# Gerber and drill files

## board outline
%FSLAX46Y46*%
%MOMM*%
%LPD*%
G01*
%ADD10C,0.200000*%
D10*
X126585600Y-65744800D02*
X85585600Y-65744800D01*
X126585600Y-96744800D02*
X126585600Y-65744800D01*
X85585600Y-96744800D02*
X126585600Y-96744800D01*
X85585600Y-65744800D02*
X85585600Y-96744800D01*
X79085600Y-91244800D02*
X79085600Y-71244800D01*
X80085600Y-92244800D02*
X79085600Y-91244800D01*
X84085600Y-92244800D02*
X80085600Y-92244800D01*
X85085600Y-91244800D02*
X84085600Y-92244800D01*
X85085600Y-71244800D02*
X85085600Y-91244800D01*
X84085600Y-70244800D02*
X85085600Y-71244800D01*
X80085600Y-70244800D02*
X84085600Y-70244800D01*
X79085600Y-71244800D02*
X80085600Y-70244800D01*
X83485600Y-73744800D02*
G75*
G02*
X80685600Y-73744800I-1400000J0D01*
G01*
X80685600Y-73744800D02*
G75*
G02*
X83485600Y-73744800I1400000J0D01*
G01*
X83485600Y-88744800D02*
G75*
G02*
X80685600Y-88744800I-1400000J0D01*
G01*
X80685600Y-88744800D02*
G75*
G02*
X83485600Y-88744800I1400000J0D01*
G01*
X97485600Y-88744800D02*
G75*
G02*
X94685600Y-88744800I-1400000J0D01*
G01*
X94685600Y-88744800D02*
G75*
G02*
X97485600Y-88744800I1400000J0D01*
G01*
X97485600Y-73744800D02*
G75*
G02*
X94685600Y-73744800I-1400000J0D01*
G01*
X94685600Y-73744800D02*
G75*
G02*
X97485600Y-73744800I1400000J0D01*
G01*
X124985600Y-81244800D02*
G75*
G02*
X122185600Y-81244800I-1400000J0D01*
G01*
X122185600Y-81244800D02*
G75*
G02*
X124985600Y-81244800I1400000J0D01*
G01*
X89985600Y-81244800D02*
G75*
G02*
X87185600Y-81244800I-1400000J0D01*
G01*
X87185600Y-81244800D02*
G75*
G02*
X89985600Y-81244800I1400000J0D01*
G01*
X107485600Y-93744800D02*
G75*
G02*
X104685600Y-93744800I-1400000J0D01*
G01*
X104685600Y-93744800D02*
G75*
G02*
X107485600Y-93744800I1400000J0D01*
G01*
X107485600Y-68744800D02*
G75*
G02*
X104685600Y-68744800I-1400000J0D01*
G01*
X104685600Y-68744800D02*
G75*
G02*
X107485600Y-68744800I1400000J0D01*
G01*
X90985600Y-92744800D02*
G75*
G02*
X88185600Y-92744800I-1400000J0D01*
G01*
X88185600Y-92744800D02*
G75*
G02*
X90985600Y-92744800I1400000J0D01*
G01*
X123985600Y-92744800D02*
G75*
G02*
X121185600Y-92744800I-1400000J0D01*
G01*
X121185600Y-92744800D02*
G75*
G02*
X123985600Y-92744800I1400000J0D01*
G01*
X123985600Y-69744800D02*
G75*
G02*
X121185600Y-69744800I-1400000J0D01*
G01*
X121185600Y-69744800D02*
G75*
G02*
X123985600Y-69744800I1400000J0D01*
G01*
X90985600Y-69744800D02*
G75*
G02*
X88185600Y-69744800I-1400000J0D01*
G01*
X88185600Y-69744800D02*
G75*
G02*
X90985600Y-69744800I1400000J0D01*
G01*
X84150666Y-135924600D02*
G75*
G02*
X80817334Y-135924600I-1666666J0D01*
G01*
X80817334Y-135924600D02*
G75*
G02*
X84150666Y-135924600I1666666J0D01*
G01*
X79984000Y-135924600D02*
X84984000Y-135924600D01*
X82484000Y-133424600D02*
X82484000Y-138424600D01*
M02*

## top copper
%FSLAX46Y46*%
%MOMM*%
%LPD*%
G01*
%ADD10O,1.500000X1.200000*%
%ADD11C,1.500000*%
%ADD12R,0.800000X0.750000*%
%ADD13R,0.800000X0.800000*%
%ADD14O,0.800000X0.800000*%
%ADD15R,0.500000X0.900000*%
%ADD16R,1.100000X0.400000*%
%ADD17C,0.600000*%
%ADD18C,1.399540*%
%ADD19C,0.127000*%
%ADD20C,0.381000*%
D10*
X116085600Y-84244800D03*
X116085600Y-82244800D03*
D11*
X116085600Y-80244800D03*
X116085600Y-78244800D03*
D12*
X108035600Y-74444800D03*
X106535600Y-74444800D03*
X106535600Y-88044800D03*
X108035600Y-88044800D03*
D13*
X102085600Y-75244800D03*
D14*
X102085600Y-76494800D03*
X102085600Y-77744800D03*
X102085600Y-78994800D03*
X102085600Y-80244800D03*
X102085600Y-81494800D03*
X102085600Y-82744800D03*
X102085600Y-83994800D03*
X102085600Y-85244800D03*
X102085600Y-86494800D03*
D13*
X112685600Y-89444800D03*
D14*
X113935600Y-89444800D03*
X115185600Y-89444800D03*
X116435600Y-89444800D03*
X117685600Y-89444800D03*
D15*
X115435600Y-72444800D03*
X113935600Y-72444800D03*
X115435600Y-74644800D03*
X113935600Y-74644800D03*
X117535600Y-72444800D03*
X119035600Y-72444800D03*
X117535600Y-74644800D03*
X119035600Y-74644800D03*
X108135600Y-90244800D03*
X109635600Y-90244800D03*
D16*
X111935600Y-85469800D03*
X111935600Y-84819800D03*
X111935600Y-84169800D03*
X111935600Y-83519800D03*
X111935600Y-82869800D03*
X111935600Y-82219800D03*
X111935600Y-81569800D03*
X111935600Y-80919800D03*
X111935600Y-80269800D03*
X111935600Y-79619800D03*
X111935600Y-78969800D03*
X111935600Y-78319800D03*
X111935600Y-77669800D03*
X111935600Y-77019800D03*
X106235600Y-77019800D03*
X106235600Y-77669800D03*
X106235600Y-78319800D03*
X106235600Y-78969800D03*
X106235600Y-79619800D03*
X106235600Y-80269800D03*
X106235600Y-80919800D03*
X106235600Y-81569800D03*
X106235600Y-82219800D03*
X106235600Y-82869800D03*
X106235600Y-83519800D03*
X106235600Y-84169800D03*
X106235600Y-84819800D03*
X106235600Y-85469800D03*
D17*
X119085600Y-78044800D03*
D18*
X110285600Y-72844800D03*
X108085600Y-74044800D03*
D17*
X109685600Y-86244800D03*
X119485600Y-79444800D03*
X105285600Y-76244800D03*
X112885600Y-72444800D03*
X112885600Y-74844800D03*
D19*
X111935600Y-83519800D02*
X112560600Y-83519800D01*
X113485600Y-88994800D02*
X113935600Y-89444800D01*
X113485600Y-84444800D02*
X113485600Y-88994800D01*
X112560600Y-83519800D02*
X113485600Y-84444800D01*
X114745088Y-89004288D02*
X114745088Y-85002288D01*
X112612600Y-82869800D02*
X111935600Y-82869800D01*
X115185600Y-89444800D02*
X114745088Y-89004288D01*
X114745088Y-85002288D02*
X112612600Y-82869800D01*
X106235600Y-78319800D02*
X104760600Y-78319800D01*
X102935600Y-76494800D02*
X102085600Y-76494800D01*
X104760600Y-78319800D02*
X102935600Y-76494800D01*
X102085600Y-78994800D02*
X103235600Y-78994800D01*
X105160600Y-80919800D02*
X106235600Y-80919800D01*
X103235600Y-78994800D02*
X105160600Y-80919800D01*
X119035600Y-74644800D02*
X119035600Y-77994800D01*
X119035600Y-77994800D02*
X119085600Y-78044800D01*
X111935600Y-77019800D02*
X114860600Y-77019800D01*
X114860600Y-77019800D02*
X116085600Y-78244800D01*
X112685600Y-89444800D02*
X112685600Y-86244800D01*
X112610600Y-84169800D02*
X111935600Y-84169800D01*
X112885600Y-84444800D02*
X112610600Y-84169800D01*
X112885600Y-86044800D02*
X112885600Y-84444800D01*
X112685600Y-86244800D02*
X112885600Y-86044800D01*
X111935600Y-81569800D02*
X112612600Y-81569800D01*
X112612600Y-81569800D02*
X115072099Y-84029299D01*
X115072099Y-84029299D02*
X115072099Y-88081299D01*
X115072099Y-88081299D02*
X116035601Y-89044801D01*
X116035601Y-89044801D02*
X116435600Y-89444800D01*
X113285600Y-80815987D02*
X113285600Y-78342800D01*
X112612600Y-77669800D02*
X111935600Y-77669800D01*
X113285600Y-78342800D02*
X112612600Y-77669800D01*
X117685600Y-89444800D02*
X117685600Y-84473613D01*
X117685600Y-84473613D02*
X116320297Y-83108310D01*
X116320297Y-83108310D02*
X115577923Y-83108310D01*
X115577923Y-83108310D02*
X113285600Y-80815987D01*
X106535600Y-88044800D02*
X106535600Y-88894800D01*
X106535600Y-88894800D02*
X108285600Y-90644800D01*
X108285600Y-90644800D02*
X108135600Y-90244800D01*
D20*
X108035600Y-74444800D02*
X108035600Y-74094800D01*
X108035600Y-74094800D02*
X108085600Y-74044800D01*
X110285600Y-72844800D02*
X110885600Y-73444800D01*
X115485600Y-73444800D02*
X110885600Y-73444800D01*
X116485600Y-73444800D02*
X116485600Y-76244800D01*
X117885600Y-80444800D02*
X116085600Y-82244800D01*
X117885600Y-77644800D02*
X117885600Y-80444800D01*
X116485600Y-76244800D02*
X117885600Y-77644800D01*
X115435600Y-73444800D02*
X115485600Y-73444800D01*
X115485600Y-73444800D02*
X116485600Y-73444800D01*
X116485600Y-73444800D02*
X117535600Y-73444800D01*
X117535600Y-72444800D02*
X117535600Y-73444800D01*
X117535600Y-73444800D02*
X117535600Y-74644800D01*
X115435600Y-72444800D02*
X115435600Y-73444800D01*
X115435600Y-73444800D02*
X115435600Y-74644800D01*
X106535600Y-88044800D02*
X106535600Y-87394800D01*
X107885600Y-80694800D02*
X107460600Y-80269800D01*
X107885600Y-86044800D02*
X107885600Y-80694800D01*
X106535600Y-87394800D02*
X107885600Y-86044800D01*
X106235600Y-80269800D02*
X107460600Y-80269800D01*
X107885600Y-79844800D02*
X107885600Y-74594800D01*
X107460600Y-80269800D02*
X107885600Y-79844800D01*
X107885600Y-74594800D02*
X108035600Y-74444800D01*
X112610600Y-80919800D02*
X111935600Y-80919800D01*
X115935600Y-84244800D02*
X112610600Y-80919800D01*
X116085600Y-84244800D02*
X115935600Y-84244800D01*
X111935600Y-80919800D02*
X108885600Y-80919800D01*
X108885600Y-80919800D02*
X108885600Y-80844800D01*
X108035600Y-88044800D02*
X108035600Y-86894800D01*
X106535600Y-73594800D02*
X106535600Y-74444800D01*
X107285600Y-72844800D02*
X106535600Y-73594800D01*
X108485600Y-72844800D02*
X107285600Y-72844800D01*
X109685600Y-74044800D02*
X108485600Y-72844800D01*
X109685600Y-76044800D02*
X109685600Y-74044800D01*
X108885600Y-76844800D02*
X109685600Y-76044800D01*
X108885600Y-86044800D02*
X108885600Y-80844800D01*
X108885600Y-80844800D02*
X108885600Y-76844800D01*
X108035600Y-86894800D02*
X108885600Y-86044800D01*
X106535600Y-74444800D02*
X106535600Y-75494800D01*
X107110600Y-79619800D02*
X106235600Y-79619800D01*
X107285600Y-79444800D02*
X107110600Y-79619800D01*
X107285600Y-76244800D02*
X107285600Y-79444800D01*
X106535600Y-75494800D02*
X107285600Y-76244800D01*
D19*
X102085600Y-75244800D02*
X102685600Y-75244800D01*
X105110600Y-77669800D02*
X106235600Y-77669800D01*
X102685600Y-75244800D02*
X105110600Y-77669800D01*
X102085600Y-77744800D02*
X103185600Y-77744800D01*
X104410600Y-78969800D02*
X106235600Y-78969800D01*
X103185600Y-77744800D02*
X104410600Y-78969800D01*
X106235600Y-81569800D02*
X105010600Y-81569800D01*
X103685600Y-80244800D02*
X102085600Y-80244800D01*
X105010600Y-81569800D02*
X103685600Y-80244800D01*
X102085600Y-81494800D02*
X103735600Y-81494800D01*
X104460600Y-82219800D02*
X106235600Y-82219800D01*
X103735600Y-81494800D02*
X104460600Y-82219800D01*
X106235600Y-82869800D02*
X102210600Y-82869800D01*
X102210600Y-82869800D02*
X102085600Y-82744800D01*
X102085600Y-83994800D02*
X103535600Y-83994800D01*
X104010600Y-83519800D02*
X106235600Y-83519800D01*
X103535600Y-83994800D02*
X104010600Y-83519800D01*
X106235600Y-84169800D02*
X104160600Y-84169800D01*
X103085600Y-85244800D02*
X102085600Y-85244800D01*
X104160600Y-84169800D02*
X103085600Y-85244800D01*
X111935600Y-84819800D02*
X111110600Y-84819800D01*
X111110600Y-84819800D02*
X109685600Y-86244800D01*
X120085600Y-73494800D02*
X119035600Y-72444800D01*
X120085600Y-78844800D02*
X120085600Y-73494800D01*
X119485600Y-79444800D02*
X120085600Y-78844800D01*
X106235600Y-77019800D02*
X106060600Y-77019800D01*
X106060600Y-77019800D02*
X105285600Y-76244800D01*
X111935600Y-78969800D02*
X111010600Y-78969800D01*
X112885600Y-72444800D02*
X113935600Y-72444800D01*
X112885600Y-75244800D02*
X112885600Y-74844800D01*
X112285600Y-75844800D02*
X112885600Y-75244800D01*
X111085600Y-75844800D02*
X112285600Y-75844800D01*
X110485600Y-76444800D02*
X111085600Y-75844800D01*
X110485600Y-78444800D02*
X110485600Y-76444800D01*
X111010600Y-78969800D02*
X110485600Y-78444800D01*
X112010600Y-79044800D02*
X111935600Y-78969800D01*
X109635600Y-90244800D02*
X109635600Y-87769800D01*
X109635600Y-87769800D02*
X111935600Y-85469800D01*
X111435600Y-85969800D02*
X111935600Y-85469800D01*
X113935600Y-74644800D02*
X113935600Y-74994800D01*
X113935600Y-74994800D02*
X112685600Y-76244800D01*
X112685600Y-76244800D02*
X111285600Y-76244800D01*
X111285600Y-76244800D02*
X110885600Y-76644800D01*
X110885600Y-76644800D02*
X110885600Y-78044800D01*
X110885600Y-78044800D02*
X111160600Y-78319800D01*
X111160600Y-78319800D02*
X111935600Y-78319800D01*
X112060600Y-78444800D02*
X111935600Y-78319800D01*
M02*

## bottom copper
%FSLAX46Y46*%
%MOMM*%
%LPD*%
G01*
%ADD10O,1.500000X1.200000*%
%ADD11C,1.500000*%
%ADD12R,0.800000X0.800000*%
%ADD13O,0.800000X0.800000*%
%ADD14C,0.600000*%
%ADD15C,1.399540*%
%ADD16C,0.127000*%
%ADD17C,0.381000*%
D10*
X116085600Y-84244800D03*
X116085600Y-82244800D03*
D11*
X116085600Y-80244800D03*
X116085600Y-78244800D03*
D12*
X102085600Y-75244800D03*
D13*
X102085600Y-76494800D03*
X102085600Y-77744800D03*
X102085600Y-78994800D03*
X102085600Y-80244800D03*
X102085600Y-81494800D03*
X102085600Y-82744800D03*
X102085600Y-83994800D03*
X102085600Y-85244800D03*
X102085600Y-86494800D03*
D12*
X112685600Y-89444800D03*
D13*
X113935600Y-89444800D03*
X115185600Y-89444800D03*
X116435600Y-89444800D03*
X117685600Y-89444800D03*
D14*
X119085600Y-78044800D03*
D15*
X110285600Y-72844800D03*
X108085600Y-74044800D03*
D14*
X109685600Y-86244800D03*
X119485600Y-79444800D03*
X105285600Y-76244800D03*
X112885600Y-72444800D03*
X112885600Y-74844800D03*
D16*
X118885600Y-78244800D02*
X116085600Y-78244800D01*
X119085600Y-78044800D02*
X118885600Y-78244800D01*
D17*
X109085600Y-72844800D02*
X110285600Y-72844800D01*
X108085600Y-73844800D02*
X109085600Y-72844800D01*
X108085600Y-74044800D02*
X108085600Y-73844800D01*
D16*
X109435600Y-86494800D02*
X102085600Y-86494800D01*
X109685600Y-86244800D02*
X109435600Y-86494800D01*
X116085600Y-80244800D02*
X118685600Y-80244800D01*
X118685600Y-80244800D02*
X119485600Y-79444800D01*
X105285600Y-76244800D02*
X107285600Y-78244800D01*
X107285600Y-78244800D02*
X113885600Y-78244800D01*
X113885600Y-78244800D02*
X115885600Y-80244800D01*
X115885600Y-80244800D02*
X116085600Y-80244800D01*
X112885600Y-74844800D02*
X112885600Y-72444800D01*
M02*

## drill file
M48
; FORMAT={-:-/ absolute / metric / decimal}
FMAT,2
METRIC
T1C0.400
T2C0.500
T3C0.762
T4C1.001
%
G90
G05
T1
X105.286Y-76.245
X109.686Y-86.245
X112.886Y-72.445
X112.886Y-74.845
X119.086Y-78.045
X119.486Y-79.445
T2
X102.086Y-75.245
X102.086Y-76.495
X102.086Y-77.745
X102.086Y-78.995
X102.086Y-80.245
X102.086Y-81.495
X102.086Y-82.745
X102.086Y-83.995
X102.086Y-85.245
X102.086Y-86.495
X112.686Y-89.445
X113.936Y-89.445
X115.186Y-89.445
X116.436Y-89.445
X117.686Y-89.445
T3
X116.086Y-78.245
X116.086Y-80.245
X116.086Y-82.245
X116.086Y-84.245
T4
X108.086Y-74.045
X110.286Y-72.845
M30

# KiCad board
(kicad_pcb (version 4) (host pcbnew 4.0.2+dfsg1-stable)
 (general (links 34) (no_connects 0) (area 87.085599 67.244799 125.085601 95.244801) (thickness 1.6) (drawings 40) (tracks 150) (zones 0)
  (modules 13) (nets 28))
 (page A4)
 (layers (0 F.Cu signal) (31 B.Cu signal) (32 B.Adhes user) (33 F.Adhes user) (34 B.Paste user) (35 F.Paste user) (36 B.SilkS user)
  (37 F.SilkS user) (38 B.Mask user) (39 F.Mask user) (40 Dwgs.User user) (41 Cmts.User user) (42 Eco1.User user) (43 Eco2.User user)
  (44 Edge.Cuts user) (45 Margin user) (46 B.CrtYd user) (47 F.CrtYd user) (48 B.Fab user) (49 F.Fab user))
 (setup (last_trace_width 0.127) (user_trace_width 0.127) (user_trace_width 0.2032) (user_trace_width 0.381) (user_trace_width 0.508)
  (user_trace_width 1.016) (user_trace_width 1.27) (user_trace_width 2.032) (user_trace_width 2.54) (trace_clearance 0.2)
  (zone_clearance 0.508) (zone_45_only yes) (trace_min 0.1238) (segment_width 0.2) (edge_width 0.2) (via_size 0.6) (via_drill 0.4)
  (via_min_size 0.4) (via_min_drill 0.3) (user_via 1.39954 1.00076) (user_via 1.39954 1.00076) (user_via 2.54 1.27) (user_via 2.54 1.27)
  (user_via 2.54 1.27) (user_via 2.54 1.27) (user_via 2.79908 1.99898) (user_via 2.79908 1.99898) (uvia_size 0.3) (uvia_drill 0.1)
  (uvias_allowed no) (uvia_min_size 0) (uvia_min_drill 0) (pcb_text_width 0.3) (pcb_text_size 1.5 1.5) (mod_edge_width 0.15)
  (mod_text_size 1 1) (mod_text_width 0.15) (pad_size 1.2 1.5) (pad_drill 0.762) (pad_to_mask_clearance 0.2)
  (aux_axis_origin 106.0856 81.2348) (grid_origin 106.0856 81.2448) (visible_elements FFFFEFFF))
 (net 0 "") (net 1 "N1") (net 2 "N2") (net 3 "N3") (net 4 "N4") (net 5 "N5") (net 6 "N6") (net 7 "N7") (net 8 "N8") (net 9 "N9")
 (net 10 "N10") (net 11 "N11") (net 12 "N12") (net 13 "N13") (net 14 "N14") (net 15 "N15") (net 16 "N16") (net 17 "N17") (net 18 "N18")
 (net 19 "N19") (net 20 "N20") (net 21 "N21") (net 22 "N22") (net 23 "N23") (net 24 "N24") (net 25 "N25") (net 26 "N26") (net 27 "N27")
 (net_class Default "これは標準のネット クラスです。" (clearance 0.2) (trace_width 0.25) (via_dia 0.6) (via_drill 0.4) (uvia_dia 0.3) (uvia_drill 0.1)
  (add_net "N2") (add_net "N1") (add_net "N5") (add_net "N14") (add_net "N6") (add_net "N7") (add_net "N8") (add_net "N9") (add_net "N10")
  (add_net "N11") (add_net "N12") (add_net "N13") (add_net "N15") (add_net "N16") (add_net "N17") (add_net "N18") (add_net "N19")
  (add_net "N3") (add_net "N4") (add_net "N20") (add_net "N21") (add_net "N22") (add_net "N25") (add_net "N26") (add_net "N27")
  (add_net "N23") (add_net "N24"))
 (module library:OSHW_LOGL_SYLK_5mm (layer F.Cu) (at 82.0856 81.2448 270)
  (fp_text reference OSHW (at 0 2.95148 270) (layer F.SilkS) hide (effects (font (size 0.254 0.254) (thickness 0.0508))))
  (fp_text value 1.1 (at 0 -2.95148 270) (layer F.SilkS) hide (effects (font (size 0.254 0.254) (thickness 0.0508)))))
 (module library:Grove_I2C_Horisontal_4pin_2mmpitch (layer F.Cu) (at 116.0856 81.2448 90)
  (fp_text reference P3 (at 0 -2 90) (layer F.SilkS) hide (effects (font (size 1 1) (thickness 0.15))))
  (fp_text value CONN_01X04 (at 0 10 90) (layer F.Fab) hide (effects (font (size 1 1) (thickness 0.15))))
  (pad 1 thru_hole oval (at -3 0 90) (size 1.2 1.5) (drill 0.762) (layers *.Cu *.Mask F.SilkS) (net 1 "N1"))
  (pad 2 thru_hole oval (at -1 0 90) (size 1.2 1.5) (drill 0.762) (layers *.Cu *.Mask F.SilkS) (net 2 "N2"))
  (pad 3 thru_hole circle (at 1 0 90) (size 1.5 1.5) (drill 0.762) (layers *.Cu *.Mask F.SilkS) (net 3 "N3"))
  (pad 4 thru_hole circle (at 3 0 90) (size 1.5 1.5) (drill 0.762) (layers *.Cu *.Mask F.SilkS) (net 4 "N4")))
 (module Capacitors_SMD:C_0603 (layer F.Cu) (at 107.2856 74.4448 180)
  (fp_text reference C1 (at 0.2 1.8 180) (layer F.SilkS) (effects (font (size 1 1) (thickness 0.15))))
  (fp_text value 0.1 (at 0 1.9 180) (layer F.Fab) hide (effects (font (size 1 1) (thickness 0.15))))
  (pad 1 smd rect (at -0.75 0 180) (size 0.8 0.75) (layers F.Cu F.Paste F.Mask) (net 2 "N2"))
  (pad 2 smd rect (at 0.75 0 180) (size 0.8 0.75) (layers F.Cu F.Paste F.Mask) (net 1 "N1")))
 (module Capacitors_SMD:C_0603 (layer F.Cu) (at 107.2856 88.0448)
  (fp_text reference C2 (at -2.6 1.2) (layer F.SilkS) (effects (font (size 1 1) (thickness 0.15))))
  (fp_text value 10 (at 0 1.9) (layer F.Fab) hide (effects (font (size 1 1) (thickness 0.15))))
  (pad 1 smd rect (at -0.75 0) (size 0.8 0.75) (layers F.Cu F.Paste F.Mask) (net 2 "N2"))
  (pad 2 smd rect (at 0.75 0) (size 0.8 0.75) (layers F.Cu F.Paste F.Mask) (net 1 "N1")))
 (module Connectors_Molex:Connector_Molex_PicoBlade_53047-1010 (layer F.Cu) (at 102.0856 75.2448 270)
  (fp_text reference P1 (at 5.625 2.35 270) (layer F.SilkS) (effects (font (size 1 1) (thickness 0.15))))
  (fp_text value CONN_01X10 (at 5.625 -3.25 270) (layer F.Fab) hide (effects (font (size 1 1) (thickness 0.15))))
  (pad 1 thru_hole rect (at 0 0 270) (size 0.8 0.8) (drill 0.5) (layers *.Cu *.Mask F.SilkS) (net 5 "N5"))
  (pad 2 thru_hole oval (at 1.25 0 270) (size 0.8 0.8) (drill 0.5) (layers *.Cu *.Mask F.SilkS) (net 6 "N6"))
  (pad 3 thru_hole oval (at 2.5 0 270) (size 0.8 0.8) (drill 0.5) (layers *.Cu *.Mask F.SilkS) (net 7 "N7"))
  (pad 4 thru_hole oval (at 3.75 0 270) (size 0.8 0.8) (drill 0.5) (layers *.Cu *.Mask F.SilkS) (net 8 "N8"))
  (pad 5 thru_hole oval (at 5 0 270) (size 0.8 0.8) (drill 0.5) (layers *.Cu *.Mask F.SilkS) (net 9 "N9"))
  (pad 6 thru_hole oval (at 6.25 0 270) (size 0.8 0.8) (drill 0.5) (layers *.Cu *.Mask F.SilkS) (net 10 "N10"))
  (pad 7 thru_hole oval (at 7.5 0 270) (size 0.8 0.8) (drill 0.5) (layers *.Cu *.Mask F.SilkS) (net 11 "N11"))
  (pad 8 thru_hole oval (at 8.75 0 270) (size 0.8 0.8) (drill 0.5) (layers *.Cu *.Mask F.SilkS) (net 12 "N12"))
  (pad 9 thru_hole oval (at 10 0 270) (size 0.8 0.8) (drill 0.5) (layers *.Cu *.Mask F.SilkS) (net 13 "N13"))
  (pad 10 thru_hole oval (at 11.25 0 270) (size 0.8 0.8) (drill 0.5) (layers *.Cu *.Mask F.SilkS) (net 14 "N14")))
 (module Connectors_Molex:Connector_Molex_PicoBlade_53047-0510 (layer F.Cu) (at 112.6856 89.4448)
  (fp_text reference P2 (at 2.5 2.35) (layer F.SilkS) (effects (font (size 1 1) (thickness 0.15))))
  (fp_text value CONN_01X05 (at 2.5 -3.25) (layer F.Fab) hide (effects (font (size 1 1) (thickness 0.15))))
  (pad 1 thru_hole rect (at 0 0) (size 0.8 0.8) (drill 0.5) (layers *.Cu *.Mask F.SilkS) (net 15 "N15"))
  (pad 2 thru_hole oval (at 1.25 0) (size 0.8 0.8) (drill 0.5) (layers *.Cu *.Mask F.SilkS) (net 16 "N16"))
  (pad 3 thru_hole oval (at 2.5 0) (size 0.8 0.8) (drill 0.5) (layers *.Cu *.Mask F.SilkS) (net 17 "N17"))
  (pad 4 thru_hole oval (at 3.75 0) (size 0.8 0.8) (drill 0.5) (layers *.Cu *.Mask F.SilkS) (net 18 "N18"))
  (pad 5 thru_hole oval (at 5 0) (size 0.8 0.8) (drill 0.5) (layers *.Cu *.Mask F.SilkS) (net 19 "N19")))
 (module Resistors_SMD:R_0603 (layer F.Cu) (at 114.6856 72.4448 180)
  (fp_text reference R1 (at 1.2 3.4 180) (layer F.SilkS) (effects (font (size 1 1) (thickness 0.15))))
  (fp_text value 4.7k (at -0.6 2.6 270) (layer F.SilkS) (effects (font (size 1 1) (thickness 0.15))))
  (pad 1 smd rect (at -0.75 0 180) (size 0.5 0.9) (layers F.Cu F.Paste F.Mask) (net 2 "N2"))
  (pad 2 smd rect (at 0.75 0 180) (size 0.5 0.9) (layers F.Cu F.Paste F.Mask) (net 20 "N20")))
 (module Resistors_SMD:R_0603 (layer F.Cu) (at 114.6856 74.6448 180)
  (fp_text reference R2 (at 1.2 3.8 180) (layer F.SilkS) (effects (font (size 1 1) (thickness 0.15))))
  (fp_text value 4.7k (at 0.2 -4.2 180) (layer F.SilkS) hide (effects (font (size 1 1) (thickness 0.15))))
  (pad 1 smd rect (at -0.75 0 180) (size 0.5 0.9) (layers F.Cu F.Paste F.Mask) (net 2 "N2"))
  (pad 2 smd rect (at 0.75 0 180) (size 0.5 0.9) (layers F.Cu F.Paste F.Mask) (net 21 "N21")))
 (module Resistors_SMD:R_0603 (layer F.Cu) (at 118.2856 72.4448)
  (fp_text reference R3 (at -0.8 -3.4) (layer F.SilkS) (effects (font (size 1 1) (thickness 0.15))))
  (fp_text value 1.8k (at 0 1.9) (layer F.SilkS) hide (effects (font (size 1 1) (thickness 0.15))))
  (pad 1 smd rect (at -0.75 0) (size 0.5 0.9) (layers F.Cu F.Paste F.Mask) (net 2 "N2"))
  (pad 2 smd rect (at 0.75 0) (size 0.5 0.9) (layers F.Cu F.Paste F.Mask) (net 3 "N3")))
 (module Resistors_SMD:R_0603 (layer F.Cu) (at 118.2856 74.6448)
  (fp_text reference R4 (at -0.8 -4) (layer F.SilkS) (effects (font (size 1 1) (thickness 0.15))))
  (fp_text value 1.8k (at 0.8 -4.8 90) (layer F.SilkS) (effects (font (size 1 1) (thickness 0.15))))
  (pad 1 smd rect (at -0.75 0) (size 0.5 0.9) (layers F.Cu F.Paste F.Mask) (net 2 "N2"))
  (pad 2 smd rect (at 0.75 0) (size 0.5 0.9) (layers F.Cu F.Paste F.Mask) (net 4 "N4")))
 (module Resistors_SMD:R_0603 (layer F.Cu) (at 108.8856 90.2448)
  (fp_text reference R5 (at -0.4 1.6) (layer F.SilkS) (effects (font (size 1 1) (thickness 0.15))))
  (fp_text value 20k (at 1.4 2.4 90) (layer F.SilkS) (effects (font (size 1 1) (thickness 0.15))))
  (pad 1 smd rect (at -0.75 0) (size 0.5 0.9) (layers F.Cu F.Paste F.Mask) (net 2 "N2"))
  (pad 2 smd rect (at 0.75 0) (size 0.5 0.9) (layers F.Cu F.Paste F.Mask) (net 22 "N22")))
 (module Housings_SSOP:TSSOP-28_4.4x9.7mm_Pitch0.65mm (layer F.Cu) (at 109.0856 81.2448 180)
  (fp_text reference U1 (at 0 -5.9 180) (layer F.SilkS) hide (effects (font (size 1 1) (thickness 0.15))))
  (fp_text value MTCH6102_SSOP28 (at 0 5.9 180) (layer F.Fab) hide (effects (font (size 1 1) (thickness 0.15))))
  (pad 1 smd rect (at -2.85 -4.225 180) (size 1.1 0.4) (layers F.Cu F.Paste F.Mask) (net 22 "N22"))
  (pad 2 smd rect (at -2.85 -3.575 180) (size 1.1 0.4) (layers F.Cu F.Paste F.Mask) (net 14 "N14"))
  (pad 3 smd rect (at -2.85 -2.925 180) (size 1.1 0.4) (layers F.Cu F.Paste F.Mask) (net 15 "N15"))
  (pad 4 smd rect (at -2.85 -2.275 180) (size 1.1 0.4) (layers F.Cu F.Paste F.Mask) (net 16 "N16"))
  (pad 5 smd rect (at -2.85 -1.625 180) (size 1.1 0.4) (layers F.Cu F.Paste F.Mask) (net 17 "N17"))
  (pad 6 smd rect (at -2.85 -0.975 180) (size 1.1 0.4) (layers F.Cu F.Paste F.Mask) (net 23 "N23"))
  (pad 7 smd rect (at -2.85 -0.325 180) (size 1.1 0.4) (layers F.Cu F.Paste F.Mask) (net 18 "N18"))
  (pad 8 smd rect (at -2.85 0.325 180) (size 1.1 0.4) (layers F.Cu F.Paste F.Mask) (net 1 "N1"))
  (pad 9 smd rect (at -2.85 0.975 180) (size 1.1 0.4) (layers F.Cu F.Paste F.Mask) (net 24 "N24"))
  (pad 10 smd rect (at -2.85 1.625 180) (size 1.1 0.4) (layers F.Cu F.Paste F.Mask) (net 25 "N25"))
  (pad 11 smd rect (at -2.85 2.275 180) (size 1.1 0.4) (layers F.Cu F.Paste F.Mask) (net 20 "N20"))
  (pad 12 smd rect (at -2.85 2.925 180) (size 1.1 0.4) (layers F.Cu F.Paste F.Mask) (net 21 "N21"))
  (pad 13 smd rect (at -2.85 3.575 180) (size 1.1 0.4) (layers F.Cu F.Paste F.Mask) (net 19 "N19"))
  (pad 14 smd rect (at -2.85 4.225 180) (size 1.1 0.4) (layers F.Cu F.Paste F.Mask) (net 4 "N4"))
  (pad 15 smd rect (at 2.85 4.225 180) (size 1.1 0.4) (layers F.Cu F.Paste F.Mask) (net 3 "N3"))
  (pad 16 smd rect (at 2.85 3.575 180) (size 1.1 0.4) (layers F.Cu F.Paste F.Mask) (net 5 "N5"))
  (pad 17 smd rect (at 2.85 2.925 180) (size 1.1 0.4) (layers F.Cu F.Paste F.Mask) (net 6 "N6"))
  (pad 18 smd rect (at 2.85 2.275 180) (size 1.1 0.4) (layers F.Cu F.Paste F.Mask) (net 7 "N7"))
  (pad 19 smd rect (at 2.85 1.625 180) (size 1.1 0.4) (layers F.Cu F.Paste F.Mask) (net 1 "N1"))
  (pad 20 smd rect (at 2.85 0.975 180) (size 1.1 0.4) (layers F.Cu F.Paste F.Mask) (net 2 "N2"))
  (pad 21 smd rect (at 2.85 0.325 180) (size 1.1 0.4) (layers F.Cu F.Paste F.Mask) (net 8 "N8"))
  (pad 22 smd rect (at 2.85 -0.325 180) (size 1.1 0.4) (layers F.Cu F.Paste F.Mask) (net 9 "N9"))
  (pad 23 smd rect (at 2.85 -0.975 180) (size 1.1 0.4) (layers F.Cu F.Paste F.Mask) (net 10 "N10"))
  (pad 24 smd rect (at 2.85 -1.625 180) (size 1.1 0.4) (layers F.Cu F.Paste F.Mask) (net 11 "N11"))
  (pad 25 smd rect (at 2.85 -2.275 180) (size 1.1 0.4) (layers F.Cu F.Paste F.Mask) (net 12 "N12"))
  (pad 26 smd rect (at 2.85 -2.925 180) (size 1.1 0.4) (layers F.Cu F.Paste F.Mask) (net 13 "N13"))
  (pad 27 smd rect (at 2.85 -3.575 180) (size 1.1 0.4) (layers F.Cu F.Paste F.Mask) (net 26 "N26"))
  (pad 28 smd rect (at 2.85 -4.225 180) (size 1.1 0.4) (layers F.Cu F.Paste F.Mask) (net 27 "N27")))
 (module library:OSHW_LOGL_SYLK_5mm (layer F.Cu) (at 96.0856 81.2448 270)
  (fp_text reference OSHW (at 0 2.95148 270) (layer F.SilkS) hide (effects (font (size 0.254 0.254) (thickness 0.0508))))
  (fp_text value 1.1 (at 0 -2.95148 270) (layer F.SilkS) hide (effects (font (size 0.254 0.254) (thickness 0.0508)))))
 (gr_line (start 126.5856 65.7448) (end 85.5856 65.7448) (angle 90) (layer Edge.Cuts) (width 0.2))
 (gr_line (start 126.5856 96.7448) (end 126.5856 65.7448) (angle 90) (layer Edge.Cuts) (width 0.2))
 (gr_line (start 85.5856 96.7448) (end 126.5856 96.7448) (angle 90) (layer Edge.Cuts) (width 0.2))
 (gr_line (start 85.5856 65.7448) (end 85.5856 96.7448) (angle 90) (layer Edge.Cuts) (width 0.2))
 (gr_line (start 79.0856 91.2448) (end 79.0856 71.2448) (angle 90) (layer Edge.Cuts) (width 0.2))
 (gr_line (start 80.0856 92.2448) (end 79.0856 91.2448) (angle 90) (layer Edge.Cuts) (width 0.2))
 (gr_line (start 84.0856 92.2448) (end 80.0856 92.2448) (angle 90) (layer Edge.Cuts) (width 0.2))
 (gr_line (start 85.0856 91.2448) (end 84.0856 92.2448) (angle 90) (layer Edge.Cuts) (width 0.2))
 (gr_line (start 85.0856 71.2448) (end 85.0856 91.2448) (angle 90) (layer Edge.Cuts) (width 0.2))
 (gr_line (start 84.0856 70.2448) (end 85.0856 71.2448) (angle 90) (layer Edge.Cuts) (width 0.2))
 (gr_line (start 80.0856 70.2448) (end 84.0856 70.2448) (angle 90) (layer Edge.Cuts) (width 0.2))
 (gr_line (start 79.0856 71.2448) (end 80.0856 70.2448) (angle 90) (layer Edge.Cuts) (width 0.2))
 (gr_circle (center 82.0856 73.7448) (end 83.4856 73.7448) (layer Edge.Cuts) (width 0.2))
 (gr_circle (center 82.0856 88.7448) (end 83.4856 88.7448) (layer Edge.Cuts) (width 0.2))
 (gr_circle (center 96.0856 88.7448) (end 97.4856 88.7448) (layer Edge.Cuts) (width 0.2))
 (gr_circle (center 96.0856 73.7448) (end 97.4856 73.7448) (layer Edge.Cuts) (width 0.2))
 (gr_circle (center 123.5856 81.2448) (end 124.9856 81.2448) (layer Edge.Cuts) (width 0.2))
 (gr_circle (center 88.5856 81.2448) (end 89.9856 81.2448) (layer Edge.Cuts) (width 0.2))
 (gr_circle (center 106.0856 93.7448) (end 107.4856 93.7448) (layer Edge.Cuts) (width 0.2))
 (gr_circle (center 106.0856 68.7448) (end 107.4856 68.7448) (layer Edge.Cuts) (width 0.2))
 (gr_circle (center 89.5856 92.7448) (end 90.9856 92.7448) (layer Edge.Cuts) (width 0.2))
 (gr_circle (center 122.5856 92.7448) (end 123.9856 92.7448) (layer Edge.Cuts) (width 0.2))
 (gr_circle (center 122.5856 69.7448) (end 123.9856 69.7448) (layer Edge.Cuts) (width 0.2))
 (gr_circle (center 89.5856 69.7448) (end 90.9856 69.7448) (layer Edge.Cuts) (width 0.2))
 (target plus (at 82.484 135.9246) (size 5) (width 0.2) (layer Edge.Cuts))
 (segment (start 111.9356 83.5198) (end 112.5606 83.5198) (width 0.127) (layer F.Cu) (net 16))
 (segment (start 113.4856 88.9948) (end 113.9356 89.4448) (width 0.127) (layer F.Cu) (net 16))
 (segment (start 113.4856 84.4448) (end 113.4856 88.9948) (width 0.127) (layer F.Cu) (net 16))
 (segment (start 112.5606 83.5198) (end 113.4856 84.4448) (width 0.127) (layer F.Cu) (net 16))
 (segment (start 114.745088 89.004288) (end 114.745088 85.002288) (width 0.127) (layer F.Cu) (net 17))
 (segment (start 112.6126 82.8698) (end 111.9356 82.8698) (width 0.127) (layer F.Cu) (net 17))
 (segment (start 115.1856 89.4448) (end 114.745088 89.004288) (width 0.127) (layer F.Cu) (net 17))
 (segment (start 114.745088 85.002288) (end 112.6126 82.8698) (width 0.127) (layer F.Cu) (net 17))
 (segment (start 106.2356 78.3198) (end 104.7606 78.3198) (width 0.127) (layer F.Cu) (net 6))
 (segment (start 102.9356 76.4948) (end 102.0856 76.4948) (width 0.127) (layer F.Cu) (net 6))
 (segment (start 104.7606 78.3198) (end 102.9356 76.4948) (width 0.127) (layer F.Cu) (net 6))
 (segment (start 102.0856 78.9948) (end 103.2356 78.9948) (width 0.127) (layer F.Cu) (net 8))
 (segment (start 105.1606 80.9198) (end 106.2356 80.9198) (width 0.127) (layer F.Cu) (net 8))
 (segment (start 103.2356 78.9948) (end 105.1606 80.9198) (width 0.127) (layer F.Cu) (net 8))
 (segment (start 119.0356 74.6448) (end 119.0356 77.9948) (width 0.127) (layer F.Cu) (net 4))
 (segment (start 118.8856 78.2448) (end 116.0856 78.2448) (width 0.127) (layer B.Cu) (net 4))
 (segment (start 119.0856 78.0448) (end 118.8856 78.2448) (width 0.127) (layer B.Cu) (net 4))
 (via (at 119.0856 78.0448) (size 0.6) (drill 0.4) (layers F.Cu B.Cu) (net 4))
 (segment (start 119.0356 77.9948) (end 119.0856 78.0448) (width 0.127) (layer F.Cu) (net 4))
 (segment (start 111.9356 77.0198) (end 114.8606 77.0198) (width 0.127) (layer F.Cu) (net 4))
 (segment (start 114.8606 77.0198) (end 116.0856 78.2448) (width 0.127) (layer F.Cu) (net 4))
 (segment (start 112.6856 89.4448) (end 112.6856 86.2448) (width 0.127) (layer F.Cu) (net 15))
 (segment (start 112.6106 84.1698) (end 111.9356 84.1698) (width 0.127) (layer F.Cu) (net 15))
 (segment (start 112.8856 84.4448) (end 112.6106 84.1698) (width 0.127) (layer F.Cu) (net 15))
 (segment (start 112.8856 86.0448) (end 112.8856 84.4448) (width 0.127) (layer F.Cu) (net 15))
 (segment (start 112.6856 86.2448) (end 112.8856 86.0448) (width 0.127) (layer F.Cu) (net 15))
 (segment (start 111.9356 81.5698) (end 112.6126 81.5698) (width 0.127) (layer F.Cu) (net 18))
 (segment (start 112.6126 81.5698) (end 115.072099 84.029299) (width 0.127) (layer F.Cu) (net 18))
 (segment (start 115.072099 84.029299) (end 115.072099 88.081299) (width 0.127) (layer F.Cu) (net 18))
 (segment (start 115.072099 88.081299) (end 116.035601 89.044801) (width 0.127) (layer F.Cu) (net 18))
 (segment (start 116.035601 89.044801) (end 116.4356 89.4448) (width 0.127) (layer F.Cu) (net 18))
 (segment (start 113.2856 80.815987) (end 113.2856 78.3428) (width 0.127) (layer F.Cu) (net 19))
 (segment (start 112.6126 77.6698) (end 111.9356 77.6698) (width 0.127) (layer F.Cu) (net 19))
 (segment (start 113.2856 78.3428) (end 112.6126 77.6698) (width 0.127) (layer F.Cu) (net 19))
 (segment (start 117.6856 89.4448) (end 117.6856 84.473613) (width 0.127) (layer F.Cu) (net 19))
 (segment (start 117.6856 84.473613) (end 116.320297 83.10831) (width 0.127) (layer F.Cu) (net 19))
 (segment (start 116.320297 83.10831) (end 115.577923 83.10831) (width 0.127) (layer F.Cu) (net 19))
 (segment (start 115.577923 83.10831) (end 113.2856 80.815987) (width 0.127) (layer F.Cu) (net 19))
 (segment (start 106.5356 88.0448) (end 106.5356 88.8948) (width 0.127) (layer F.Cu) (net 2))
 (segment (start 106.5356 88.8948) (end 108.2856 90.6448) (width 0.127) (layer F.Cu) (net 2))
 (segment (start 108.2856 90.6448) (end 108.1356 90.2448) (width 0.127) (layer F.Cu) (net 2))
 (segment (start 108.0356 74.4448) (end 108.0356 74.0948) (width 0.381) (layer F.Cu) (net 2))
 (segment (start 108.0356 74.0948) (end 108.0856 74.0448) (width 0.381) (layer F.Cu) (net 2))
 (segment (start 110.2856 72.8448) (end 110.8856 73.4448) (width 0.381) (layer F.Cu) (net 2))
 (via (at 110.2856 72.8448) (size 1.39954) (drill 1.00076) (layers F.Cu B.Cu) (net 2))
 (segment (start 109.0856 72.8448) (end 110.2856 72.8448) (width 0.381) (layer B.Cu) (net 2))
 (segment (start 108.0856 73.8448) (end 109.0856 72.8448) (width 0.381) (layer B.Cu) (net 2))
 (segment (start 108.0856 74.0448) (end 108.0856 73.8448) (width 0.381) (layer B.Cu) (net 2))
 (via (at 108.0856 74.0448) (size 1.39954) (drill 1.00076) (layers F.Cu B.Cu) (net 2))
 (segment (start 115.4856 73.4448) (end 110.8856 73.4448) (width 0.381) (layer F.Cu) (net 2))
 (segment (start 116.4856 73.4448) (end 116.4856 76.2448) (width 0.381) (layer F.Cu) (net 2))
 (segment (start 117.8856 80.4448) (end 116.0856 82.2448) (width 0.381) (layer F.Cu) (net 2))
 (segment (start 117.8856 77.6448) (end 117.8856 80.4448) (width 0.381) (layer F.Cu) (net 2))
 (segment (start 116.4856 76.2448) (end 117.8856 77.6448) (width 0.381) (layer F.Cu) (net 2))
 (segment (start 115.4356 73.4448) (end 115.4856 73.4448) (width 0.381) (layer F.Cu) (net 2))
 (segment (start 115.4856 73.4448) (end 116.4856 73.4448) (width 0.381) (layer F.Cu) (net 2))
 (segment (start 116.4856 73.4448) (end 117.5356 73.4448) (width 0.381) (layer F.Cu) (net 2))
 (segment (start 117.5356 72.4448) (end 117.5356 73.4448) (width 0.381) (layer F.Cu) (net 2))
 (segment (start 117.5356 73.4448) (end 117.5356 74.6448) (width 0.381) (layer F.Cu) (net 2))
 (segment (start 115.4356 72.4448) (end 115.4356 73.4448) (width 0.381) (layer F.Cu) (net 2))
 (segment (start 115.4356 73.4448) (end 115.4356 74.6448) (width 0.381) (layer F.Cu) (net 2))
 (segment (start 106.5356 88.0448) (end 106.5356 87.3948) (width 0.381) (layer F.Cu) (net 2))
 (segment (start 107.8856 80.6948) (end 107.4606 80.2698) (width 0.381) (layer F.Cu) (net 2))
 (segment (start 107.8856 86.0448) (end 107.8856 80.6948) (width 0.381) (layer F.Cu) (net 2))
 (segment (start 106.5356 87.3948) (end 107.8856 86.0448) (width 0.381) (layer F.Cu) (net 2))
 (segment (start 106.2356 80.2698) (end 107.4606 80.2698) (width 0.381) (layer F.Cu) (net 2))
 (segment (start 107.8856 79.8448) (end 107.8856 74.5948) (width 0.381) (layer F.Cu) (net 2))
 (segment (start 107.4606 80.2698) (end 107.8856 79.8448) (width 0.381) (layer F.Cu) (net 2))
 (segment (start 107.8856 74.5948) (end 108.0356 74.4448) (width 0.381) (layer F.Cu) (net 2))
 (segment (start 112.6106 80.9198) (end 111.9356 80.9198) (width 0.381) (layer F.Cu) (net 1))
 (segment (start 115.9356 84.2448) (end 112.6106 80.9198) (width 0.381) (layer F.Cu) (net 1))
 (segment (start 116.0856 84.2448) (end 115.9356 84.2448) (width 0.381) (layer F.Cu) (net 1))
 (segment (start 111.9356 80.9198) (end 108.8856 80.9198) (width 0.381) (layer F.Cu) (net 1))
 (segment (start 108.8856 80.9198) (end 108.8856 80.8448) (width 0.381) (layer F.Cu) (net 1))
 (segment (start 108.0356 88.0448) (end 108.0356 86.8948) (width 0.381) (layer F.Cu) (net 1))
 (segment (start 106.5356 73.5948) (end 106.5356 74.4448) (width 0.381) (layer F.Cu) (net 1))
 (segment (start 107.2856 72.8448) (end 106.5356 73.5948) (width 0.381) (layer F.Cu) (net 1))
 (segment (start 108.4856 72.8448) (end 107.2856 72.8448) (width 0.381) (layer F.Cu) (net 1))
 (segment (start 109.6856 74.0448) (end 108.4856 72.8448) (width 0.381) (layer F.Cu) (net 1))
 (segment (start 109.6856 76.0448) (end 109.6856 74.0448) (width 0.381) (layer F.Cu) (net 1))
 (segment (start 108.8856 76.8448) (end 109.6856 76.0448) (width 0.381) (layer F.Cu) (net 1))
 (segment (start 108.8856 86.0448) (end 108.8856 80.8448) (width 0.381) (layer F.Cu) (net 1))
 (segment (start 108.8856 80.8448) (end 108.8856 76.8448) (width 0.381) (layer F.Cu) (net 1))
 (segment (start 108.0356 86.8948) (end 108.8856 86.0448) (width 0.381) (layer F.Cu) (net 1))
 (segment (start 106.5356 74.4448) (end 106.5356 75.4948) (width 0.381) (layer F.Cu) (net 1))
 (segment (start 107.1106 79.6198) (end 106.2356 79.6198) (width 0.381) (layer F.Cu) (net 1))
 (segment (start 107.2856 79.4448) (end 107.1106 79.6198) (width 0.381) (layer F.Cu) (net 1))
 (segment (start 107.2856 76.2448) (end 107.2856 79.4448) (width 0.381) (layer F.Cu) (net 1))
 (segment (start 106.5356 75.4948) (end 107.2856 76.2448) (width 0.381) (layer F.Cu) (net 1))
 (segment (start 102.0856 75.2448) (end 102.6856 75.2448) (width 0.127) (layer F.Cu) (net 5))
 (segment (start 105.1106 77.6698) (end 106.2356 77.6698) (width 0.127) (layer F.Cu) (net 5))
 (segment (start 102.6856 75.2448) (end 105.1106 77.6698) (width 0.127) (layer F.Cu) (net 5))
 (segment (start 102.0856 77.7448) (end 103.1856 77.7448) (width 0.127) (layer F.Cu) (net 7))
 (segment (start 104.4106 78.9698) (end 106.2356 78.9698) (width 0.127) (layer F.Cu) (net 7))
 (segment (start 103.1856 77.7448) (end 104.4106 78.9698) (width 0.127) (layer F.Cu) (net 7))
 (segment (start 106.2356 81.5698) (end 105.0106 81.5698) (width 0.127) (layer F.Cu) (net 9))
 (segment (start 103.6856 80.2448) (end 102.0856 80.2448) (width 0.127) (layer F.Cu) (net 9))
 (segment (start 105.0106 81.5698) (end 103.6856 80.2448) (width 0.127) (layer F.Cu) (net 9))
 (segment (start 102.0856 81.4948) (end 103.7356 81.4948) (width 0.127) (layer F.Cu) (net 10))
 (segment (start 104.4606 82.2198) (end 106.2356 82.2198) (width 0.127) (layer F.Cu) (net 10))
 (segment (start 103.7356 81.4948) (end 104.4606 82.2198) (width 0.127) (layer F.Cu) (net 10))
 (segment (start 106.2356 82.8698) (end 102.2106 82.8698) (width 0.127) (layer F.Cu) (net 11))
 (segment (start 102.2106 82.8698) (end 102.0856 82.7448) (width 0.127) (layer F.Cu) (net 11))
 (segment (start 102.0856 83.9948) (end 103.5356 83.9948) (width 0.127) (layer F.Cu) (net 12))
 (segment (start 104.0106 83.5198) (end 106.2356 83.5198) (width 0.127) (layer F.Cu) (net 12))
 (segment (start 103.5356 83.9948) (end 104.0106 83.5198) (width 0.127) (layer F.Cu) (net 12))
 (segment (start 106.2356 84.1698) (end 104.1606 84.1698) (width 0.127) (layer F.Cu) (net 13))
 (segment (start 103.0856 85.2448) (end 102.0856 85.2448) (width 0.127) (layer F.Cu) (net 13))
 (segment (start 104.1606 84.1698) (end 103.0856 85.2448) (width 0.127) (layer F.Cu) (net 13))
 (segment (start 111.9356 84.8198) (end 111.1106 84.8198) (width 0.127) (layer F.Cu) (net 14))
 (segment (start 109.4356 86.4948) (end 102.0856 86.4948) (width 0.127) (layer B.Cu) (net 14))
 (segment (start 109.6856 86.2448) (end 109.4356 86.4948) (width 0.127) (layer B.Cu) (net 14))
 (via (at 109.6856 86.2448) (size 0.6) (drill 0.4) (layers F.Cu B.Cu) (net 14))
 (segment (start 111.1106 84.8198) (end 109.6856 86.2448) (width 0.127) (layer F.Cu) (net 14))
 (segment (start 116.0856 80.2448) (end 118.6856 80.2448) (width 0.127) (layer B.Cu) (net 3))
 (segment (start 120.0856 73.4948) (end 119.0356 72.4448) (width 0.127) (layer F.Cu) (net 3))
 (segment (start 120.0856 78.8448) (end 120.0856 73.4948) (width 0.127) (layer F.Cu) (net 3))
 (segment (start 119.4856 79.4448) (end 120.0856 78.8448) (width 0.127) (layer F.Cu) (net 3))
 (via (at 119.4856 79.4448) (size 0.6) (drill 0.4) (layers F.Cu B.Cu) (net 3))
 (segment (start 118.6856 80.2448) (end 119.4856 79.4448) (width 0.127) (layer B.Cu) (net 3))
 (segment (start 106.2356 77.0198) (end 106.0606 77.0198) (width 0.127) (layer F.Cu) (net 3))
 (segment (start 106.0606 77.0198) (end 105.2856 76.2448) (width 0.127) (layer F.Cu) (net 3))
 (via (at 105.2856 76.2448) (size 0.6) (drill 0.4) (layers F.Cu B.Cu) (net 3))
 (segment (start 105.2856 76.2448) (end 107.2856 78.2448) (width 0.127) (layer B.Cu) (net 3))
 (segment (start 107.2856 78.2448) (end 113.8856 78.2448) (width 0.127) (layer B.Cu) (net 3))
 (segment (start 113.8856 78.2448) (end 115.8856 80.2448) (width 0.127) (layer B.Cu) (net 3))
 (segment (start 115.8856 80.2448) (end 116.0856 80.2448) (width 0.127) (layer B.Cu) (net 3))
 (segment (start 111.9356 78.9698) (end 111.0106 78.9698) (width 0.127) (layer F.Cu) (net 20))
 (segment (start 112.8856 72.4448) (end 113.9356 72.4448) (width 0.127) (layer F.Cu) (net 20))
 (via (at 112.8856 72.4448) (size 0.6) (drill 0.4) (layers F.Cu B.Cu) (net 20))
 (segment (start 112.8856 74.8448) (end 112.8856 72.4448) (width 0.127) (layer B.Cu) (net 20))
 (via (at 112.8856 74.8448) (size 0.6) (drill 0.4) (layers F.Cu B.Cu) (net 20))
 (segment (start 112.8856 75.2448) (end 112.8856 74.8448) (width 0.127) (layer F.Cu) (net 20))
 (segment (start 112.2856 75.8448) (end 112.8856 75.2448) (width 0.127) (layer F.Cu) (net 20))
 (segment (start 111.0856 75.8448) (end 112.2856 75.8448) (width 0.127) (layer F.Cu) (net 20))
 (segment (start 110.4856 76.4448) (end 111.0856 75.8448) (width 0.127) (layer F.Cu) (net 20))
 (segment (start 110.4856 78.4448) (end 110.4856 76.4448) (width 0.127) (layer F.Cu) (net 20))
 (segment (start 111.0106 78.9698) (end 110.4856 78.4448) (width 0.127) (layer F.Cu) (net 20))
 (segment (start 112.0106 79.0448) (end 111.9356 78.9698) (width 0.127) (layer F.Cu) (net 20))
 (segment (start 109.6356 90.2448) (end 109.6356 87.7698) (width 0.127) (layer F.Cu) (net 22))
 (segment (start 109.6356 87.7698) (end 111.9356 85.4698) (width 0.127) (layer F.Cu) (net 22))
 (segment (start 111.4356 85.9698) (end 111.9356 85.4698) (width 0.127) (layer F.Cu) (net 22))
 (segment (start 113.9356 74.6448) (end 113.9356 74.9948) (width 0.127) (layer F.Cu) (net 21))
 (segment (start 113.9356 74.9948) (end 112.6856 76.2448) (width 0.127) (layer F.Cu) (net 21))
 (segment (start 112.6856 76.2448) (end 111.2856 76.2448) (width 0.127) (layer F.Cu) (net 21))
 (segment (start 111.2856 76.2448) (end 110.8856 76.6448) (width 0.127) (layer F.Cu) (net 21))
 (segment (start 110.8856 76.6448) (end 110.8856 78.0448) (width 0.127) (layer F.Cu) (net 21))
 (segment (start 110.8856 78.0448) (end 111.1606 78.3198) (width 0.127) (layer F.Cu) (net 21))
 (segment (start 111.1606 78.3198) (end 111.9356 78.3198) (width 0.127) (layer F.Cu) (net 21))
 (segment (start 112.0606 78.4448) (end 111.9356 78.3198) (width 0.127) (layer F.Cu) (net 21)))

